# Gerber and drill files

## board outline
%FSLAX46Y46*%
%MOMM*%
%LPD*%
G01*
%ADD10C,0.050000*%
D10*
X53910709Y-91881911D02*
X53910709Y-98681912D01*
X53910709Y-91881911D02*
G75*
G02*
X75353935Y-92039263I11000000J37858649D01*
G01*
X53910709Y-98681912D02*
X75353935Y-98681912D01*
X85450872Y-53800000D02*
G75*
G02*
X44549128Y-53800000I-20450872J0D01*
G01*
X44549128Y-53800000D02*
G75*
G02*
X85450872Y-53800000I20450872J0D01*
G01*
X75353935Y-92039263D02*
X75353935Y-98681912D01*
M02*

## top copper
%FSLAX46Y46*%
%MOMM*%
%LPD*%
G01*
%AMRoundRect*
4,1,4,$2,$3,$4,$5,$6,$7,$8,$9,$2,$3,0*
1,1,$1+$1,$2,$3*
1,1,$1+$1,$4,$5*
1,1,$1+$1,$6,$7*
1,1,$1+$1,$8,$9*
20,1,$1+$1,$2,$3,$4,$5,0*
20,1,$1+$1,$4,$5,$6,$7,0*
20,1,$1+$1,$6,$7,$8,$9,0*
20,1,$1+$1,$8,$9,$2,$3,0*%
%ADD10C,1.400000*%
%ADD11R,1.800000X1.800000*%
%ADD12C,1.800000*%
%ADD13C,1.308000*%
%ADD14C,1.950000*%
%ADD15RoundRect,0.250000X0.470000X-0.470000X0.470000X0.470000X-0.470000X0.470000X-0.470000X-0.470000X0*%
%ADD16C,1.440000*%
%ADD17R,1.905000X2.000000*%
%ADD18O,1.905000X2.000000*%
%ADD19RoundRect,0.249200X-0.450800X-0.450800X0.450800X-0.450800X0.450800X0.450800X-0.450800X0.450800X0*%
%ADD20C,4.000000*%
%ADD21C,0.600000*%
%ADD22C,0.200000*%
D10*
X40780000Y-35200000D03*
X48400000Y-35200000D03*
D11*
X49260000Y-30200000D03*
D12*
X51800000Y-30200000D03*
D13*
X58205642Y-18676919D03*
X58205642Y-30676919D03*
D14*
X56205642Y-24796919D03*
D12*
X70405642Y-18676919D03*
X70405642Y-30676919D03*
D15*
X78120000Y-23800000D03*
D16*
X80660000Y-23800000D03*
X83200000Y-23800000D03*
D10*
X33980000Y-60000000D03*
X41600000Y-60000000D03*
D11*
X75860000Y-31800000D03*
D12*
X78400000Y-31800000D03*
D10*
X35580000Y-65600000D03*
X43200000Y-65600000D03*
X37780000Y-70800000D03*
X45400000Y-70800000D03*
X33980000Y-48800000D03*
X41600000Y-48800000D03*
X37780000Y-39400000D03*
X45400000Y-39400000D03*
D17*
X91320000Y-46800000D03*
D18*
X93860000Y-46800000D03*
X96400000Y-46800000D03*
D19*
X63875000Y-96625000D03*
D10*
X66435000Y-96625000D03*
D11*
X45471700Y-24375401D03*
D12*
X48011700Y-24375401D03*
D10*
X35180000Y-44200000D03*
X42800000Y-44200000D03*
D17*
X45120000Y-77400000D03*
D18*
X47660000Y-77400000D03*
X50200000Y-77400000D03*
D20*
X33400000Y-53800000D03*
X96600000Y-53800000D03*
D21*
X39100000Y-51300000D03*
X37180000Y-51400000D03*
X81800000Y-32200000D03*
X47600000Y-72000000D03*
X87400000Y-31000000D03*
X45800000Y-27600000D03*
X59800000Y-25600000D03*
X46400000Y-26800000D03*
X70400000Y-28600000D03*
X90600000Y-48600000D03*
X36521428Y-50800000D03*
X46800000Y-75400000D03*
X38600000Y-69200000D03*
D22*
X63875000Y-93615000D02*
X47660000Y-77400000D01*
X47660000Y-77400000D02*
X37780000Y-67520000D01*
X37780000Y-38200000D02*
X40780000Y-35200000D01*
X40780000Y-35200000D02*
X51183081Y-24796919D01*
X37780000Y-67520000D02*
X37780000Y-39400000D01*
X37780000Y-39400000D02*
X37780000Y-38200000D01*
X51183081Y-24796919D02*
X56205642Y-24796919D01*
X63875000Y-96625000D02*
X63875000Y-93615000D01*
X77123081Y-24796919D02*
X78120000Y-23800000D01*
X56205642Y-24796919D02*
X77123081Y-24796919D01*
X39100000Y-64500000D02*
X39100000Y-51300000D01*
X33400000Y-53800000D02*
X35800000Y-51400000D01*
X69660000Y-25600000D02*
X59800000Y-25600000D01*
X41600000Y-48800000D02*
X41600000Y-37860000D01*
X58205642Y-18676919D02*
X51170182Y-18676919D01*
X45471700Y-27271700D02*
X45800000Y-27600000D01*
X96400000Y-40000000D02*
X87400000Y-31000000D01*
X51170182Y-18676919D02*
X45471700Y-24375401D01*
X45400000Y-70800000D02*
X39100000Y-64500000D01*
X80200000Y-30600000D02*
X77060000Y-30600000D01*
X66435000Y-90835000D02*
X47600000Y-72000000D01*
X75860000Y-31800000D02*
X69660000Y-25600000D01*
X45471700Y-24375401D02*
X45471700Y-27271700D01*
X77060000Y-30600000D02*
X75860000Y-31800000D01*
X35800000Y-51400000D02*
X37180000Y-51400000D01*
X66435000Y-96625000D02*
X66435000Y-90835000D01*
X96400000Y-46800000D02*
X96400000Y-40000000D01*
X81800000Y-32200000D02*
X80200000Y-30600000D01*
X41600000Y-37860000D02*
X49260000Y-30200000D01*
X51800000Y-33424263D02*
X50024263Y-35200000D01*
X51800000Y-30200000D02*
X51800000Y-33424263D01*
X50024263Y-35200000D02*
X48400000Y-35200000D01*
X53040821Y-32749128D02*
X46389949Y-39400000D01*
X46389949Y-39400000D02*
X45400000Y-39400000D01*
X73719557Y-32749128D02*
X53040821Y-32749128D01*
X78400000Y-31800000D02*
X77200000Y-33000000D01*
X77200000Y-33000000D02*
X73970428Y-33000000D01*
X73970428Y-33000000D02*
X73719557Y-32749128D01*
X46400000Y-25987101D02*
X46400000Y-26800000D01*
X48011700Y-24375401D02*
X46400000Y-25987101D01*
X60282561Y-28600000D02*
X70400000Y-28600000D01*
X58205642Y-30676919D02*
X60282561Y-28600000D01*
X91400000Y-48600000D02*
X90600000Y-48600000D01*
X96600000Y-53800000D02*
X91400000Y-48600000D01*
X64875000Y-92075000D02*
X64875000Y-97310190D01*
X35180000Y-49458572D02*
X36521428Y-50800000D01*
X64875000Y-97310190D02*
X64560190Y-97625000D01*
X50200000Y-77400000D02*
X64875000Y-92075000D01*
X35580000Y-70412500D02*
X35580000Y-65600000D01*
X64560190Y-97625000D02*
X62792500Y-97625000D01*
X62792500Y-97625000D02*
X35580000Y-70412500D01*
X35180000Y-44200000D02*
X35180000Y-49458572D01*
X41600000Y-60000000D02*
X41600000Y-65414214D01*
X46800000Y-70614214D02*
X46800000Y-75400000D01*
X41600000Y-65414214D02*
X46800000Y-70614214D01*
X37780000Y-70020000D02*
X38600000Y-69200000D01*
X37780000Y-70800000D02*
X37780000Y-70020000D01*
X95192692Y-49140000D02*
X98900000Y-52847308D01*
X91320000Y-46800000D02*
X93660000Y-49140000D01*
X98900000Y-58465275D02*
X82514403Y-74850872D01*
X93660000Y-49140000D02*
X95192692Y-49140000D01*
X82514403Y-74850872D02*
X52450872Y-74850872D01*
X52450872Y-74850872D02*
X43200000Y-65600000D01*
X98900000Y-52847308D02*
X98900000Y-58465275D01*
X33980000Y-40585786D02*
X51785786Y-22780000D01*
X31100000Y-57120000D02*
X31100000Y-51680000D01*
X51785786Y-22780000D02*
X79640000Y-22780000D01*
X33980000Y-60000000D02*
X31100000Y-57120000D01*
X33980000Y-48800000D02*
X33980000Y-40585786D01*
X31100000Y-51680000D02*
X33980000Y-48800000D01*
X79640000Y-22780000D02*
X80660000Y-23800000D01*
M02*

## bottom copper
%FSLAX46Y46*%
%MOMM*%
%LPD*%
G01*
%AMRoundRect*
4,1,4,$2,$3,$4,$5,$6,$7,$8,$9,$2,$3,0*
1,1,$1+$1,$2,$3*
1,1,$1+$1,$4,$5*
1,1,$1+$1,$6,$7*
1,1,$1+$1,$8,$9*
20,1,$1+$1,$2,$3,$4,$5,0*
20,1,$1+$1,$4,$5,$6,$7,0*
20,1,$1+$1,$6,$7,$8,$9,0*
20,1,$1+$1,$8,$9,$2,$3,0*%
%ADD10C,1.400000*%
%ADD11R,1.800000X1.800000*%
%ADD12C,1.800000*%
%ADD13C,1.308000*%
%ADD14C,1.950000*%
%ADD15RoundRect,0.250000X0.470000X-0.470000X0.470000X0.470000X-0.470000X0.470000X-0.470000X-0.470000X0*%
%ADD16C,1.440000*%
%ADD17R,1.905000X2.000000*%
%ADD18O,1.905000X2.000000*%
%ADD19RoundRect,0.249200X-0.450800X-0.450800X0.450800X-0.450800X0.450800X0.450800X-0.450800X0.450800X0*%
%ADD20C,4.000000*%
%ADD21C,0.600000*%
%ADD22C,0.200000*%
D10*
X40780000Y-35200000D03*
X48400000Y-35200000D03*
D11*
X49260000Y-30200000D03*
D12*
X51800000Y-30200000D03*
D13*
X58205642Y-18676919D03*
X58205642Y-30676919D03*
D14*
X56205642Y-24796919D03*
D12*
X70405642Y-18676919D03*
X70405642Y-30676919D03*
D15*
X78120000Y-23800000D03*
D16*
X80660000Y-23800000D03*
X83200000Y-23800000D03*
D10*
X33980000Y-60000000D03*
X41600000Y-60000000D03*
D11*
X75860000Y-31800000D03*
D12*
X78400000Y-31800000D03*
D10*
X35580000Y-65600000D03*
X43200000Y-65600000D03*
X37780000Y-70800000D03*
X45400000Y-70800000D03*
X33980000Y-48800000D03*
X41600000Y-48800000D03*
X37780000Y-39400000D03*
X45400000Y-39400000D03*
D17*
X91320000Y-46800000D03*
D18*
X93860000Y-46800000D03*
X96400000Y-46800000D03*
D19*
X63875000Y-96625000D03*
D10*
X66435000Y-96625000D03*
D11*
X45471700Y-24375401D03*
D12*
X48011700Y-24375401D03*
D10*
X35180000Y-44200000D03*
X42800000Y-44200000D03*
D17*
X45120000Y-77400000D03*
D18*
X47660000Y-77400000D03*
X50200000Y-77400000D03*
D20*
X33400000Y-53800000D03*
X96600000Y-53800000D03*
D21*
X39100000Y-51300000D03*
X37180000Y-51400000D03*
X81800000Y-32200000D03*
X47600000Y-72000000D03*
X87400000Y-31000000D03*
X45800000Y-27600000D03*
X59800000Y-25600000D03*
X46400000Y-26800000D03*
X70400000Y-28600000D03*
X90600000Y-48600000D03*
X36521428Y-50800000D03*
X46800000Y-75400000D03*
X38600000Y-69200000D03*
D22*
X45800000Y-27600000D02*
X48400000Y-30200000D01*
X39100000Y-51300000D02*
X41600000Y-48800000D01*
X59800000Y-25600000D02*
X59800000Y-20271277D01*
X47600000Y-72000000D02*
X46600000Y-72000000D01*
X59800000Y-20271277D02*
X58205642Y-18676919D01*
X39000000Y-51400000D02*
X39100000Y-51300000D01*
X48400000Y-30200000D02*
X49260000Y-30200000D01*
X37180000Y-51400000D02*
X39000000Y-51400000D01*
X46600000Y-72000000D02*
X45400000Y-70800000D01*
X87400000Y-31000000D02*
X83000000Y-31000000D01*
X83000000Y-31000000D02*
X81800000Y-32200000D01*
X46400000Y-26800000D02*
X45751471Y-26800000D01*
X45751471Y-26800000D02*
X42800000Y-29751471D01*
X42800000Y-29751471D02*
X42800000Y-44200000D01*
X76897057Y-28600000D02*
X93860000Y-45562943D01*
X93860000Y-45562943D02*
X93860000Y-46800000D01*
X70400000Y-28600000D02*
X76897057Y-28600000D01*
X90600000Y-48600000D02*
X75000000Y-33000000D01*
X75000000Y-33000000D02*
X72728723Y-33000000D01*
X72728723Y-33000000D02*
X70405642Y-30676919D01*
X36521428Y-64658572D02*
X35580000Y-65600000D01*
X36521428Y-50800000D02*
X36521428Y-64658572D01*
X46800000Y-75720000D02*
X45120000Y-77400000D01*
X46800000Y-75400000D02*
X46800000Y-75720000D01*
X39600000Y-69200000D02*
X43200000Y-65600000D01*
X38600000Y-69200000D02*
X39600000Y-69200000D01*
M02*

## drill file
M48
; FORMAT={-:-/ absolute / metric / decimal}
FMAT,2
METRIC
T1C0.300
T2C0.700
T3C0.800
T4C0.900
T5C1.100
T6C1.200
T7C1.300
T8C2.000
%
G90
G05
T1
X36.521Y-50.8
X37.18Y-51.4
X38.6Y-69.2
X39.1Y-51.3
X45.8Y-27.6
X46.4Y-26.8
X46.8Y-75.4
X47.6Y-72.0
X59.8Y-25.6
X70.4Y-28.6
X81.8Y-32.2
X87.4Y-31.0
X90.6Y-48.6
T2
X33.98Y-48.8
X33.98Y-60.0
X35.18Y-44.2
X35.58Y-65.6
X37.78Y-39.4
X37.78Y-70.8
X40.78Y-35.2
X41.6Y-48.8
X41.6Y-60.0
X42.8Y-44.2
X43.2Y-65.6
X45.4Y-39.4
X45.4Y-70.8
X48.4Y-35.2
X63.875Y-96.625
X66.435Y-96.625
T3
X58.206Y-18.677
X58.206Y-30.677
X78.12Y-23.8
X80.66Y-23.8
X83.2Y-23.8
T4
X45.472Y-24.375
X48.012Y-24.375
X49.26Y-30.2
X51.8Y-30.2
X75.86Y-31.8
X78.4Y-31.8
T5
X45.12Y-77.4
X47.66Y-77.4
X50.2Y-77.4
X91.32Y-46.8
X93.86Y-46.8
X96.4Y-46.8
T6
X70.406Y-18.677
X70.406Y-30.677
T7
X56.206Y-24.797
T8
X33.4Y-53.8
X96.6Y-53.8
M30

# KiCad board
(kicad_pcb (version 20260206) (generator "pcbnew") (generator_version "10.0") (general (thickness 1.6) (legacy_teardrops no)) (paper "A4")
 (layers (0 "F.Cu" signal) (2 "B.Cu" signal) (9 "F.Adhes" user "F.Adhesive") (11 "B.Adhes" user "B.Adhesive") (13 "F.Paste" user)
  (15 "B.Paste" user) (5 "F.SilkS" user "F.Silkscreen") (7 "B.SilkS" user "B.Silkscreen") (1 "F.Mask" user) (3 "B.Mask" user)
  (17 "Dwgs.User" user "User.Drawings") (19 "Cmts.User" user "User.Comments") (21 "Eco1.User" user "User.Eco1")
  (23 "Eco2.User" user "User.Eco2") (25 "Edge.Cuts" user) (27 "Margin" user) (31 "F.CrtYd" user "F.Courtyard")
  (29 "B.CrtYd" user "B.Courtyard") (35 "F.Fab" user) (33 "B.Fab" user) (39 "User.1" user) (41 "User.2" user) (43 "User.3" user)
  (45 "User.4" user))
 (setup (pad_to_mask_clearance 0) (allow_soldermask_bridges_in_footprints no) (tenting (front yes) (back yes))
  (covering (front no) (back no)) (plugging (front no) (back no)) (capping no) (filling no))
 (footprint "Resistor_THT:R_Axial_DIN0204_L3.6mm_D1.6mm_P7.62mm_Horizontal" (layer "F.Cu") (at 40.78 35.2)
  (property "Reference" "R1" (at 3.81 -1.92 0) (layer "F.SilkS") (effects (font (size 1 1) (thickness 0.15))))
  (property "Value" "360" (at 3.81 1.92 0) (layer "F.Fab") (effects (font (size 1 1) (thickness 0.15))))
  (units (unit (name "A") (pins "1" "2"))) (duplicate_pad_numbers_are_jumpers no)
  (pad "1" thru_hole circle (at 0 0) (size 1.4 1.4) (drill 0.7) (layers "*.Cu" "*.Mask") (remove_unused_layers no) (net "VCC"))
  (pad "2" thru_hole circle (at 7.62 0) (size 1.4 1.4) (drill 0.7) (layers "*.Cu" "*.Mask") (remove_unused_layers no) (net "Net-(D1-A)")))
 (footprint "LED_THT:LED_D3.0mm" (layer "F.Cu") (at 49.26 30.2)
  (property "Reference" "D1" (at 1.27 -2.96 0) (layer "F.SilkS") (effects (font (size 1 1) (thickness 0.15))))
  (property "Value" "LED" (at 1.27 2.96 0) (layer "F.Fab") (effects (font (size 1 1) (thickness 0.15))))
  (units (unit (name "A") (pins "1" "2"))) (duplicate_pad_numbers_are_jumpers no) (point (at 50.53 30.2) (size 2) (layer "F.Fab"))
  (pad "1" thru_hole rect (at 0 0) (size 1.8 1.8) (drill 0.9) (layers "*.Cu" "*.Mask") (remove_unused_layers no) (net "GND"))
  (pad "2" thru_hole circle (at 2.54 0) (size 1.8 1.8) (drill 0.9) (layers "*.Cu" "*.Mask") (remove_unused_layers no) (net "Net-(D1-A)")))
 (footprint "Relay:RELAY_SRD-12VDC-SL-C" (layer "F.Cu") (at 64.305642 24.676919)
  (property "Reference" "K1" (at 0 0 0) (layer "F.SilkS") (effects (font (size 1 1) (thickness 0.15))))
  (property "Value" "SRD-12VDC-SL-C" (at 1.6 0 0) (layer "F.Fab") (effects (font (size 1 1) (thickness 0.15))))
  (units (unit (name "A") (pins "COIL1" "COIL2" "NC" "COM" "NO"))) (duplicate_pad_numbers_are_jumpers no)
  (pad "COIL1" thru_hole circle (at -6.1 -6) (size 1.308 1.308) (drill 0.8) (layers "*.Cu" "*.Mask") (remove_unused_layers no) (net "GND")
   (solder_mask_margin 0.102))
  (pad "COIL2" thru_hole circle (at -6.1 6) (size 1.308 1.308) (drill 0.8) (layers "*.Cu" "*.Mask") (remove_unused_layers no)
   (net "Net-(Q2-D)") (solder_mask_margin 0.102))
  (pad "COM" thru_hole circle (at -8.1 0.12) (size 1.95 1.95) (drill 1.3) (layers "*.Cu" "*.Mask") (remove_unused_layers no) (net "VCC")
   (solder_mask_margin 0.102))
  (pad "NC" thru_hole circle (at 6.1 -6) (size 1.8 1.8) (drill 1.2) (layers "*.Cu" "*.Mask") (remove_unused_layers no)
   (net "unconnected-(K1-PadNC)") (solder_mask_margin 0.102))
  (pad "NO" thru_hole circle (at 6.1 6) (size 1.8 1.8) (drill 1.2) (layers "*.Cu" "*.Mask") (remove_unused_layers no) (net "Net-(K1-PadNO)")
   (solder_mask_margin 0.102)))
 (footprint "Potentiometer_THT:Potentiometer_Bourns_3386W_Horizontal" (layer "F.Cu") (at 78.12 23.8)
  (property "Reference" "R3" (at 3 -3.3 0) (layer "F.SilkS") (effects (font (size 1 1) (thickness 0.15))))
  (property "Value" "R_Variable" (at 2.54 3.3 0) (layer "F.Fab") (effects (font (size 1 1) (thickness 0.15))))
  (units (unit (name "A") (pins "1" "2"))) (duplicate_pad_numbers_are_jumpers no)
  (pad "1" thru_hole roundrect (at 0 0 90) (size 1.44 1.44) (drill 0.8) (layers "*.Cu" "*.Mask") (remove_unused_layers no)
   (roundrect_rratio 0.1736111111) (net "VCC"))
  (pad "2" thru_hole circle (at 2.54 0 90) (size 1.44 1.44) (drill 0.8) (layers "*.Cu" "*.Mask") (remove_unused_layers no)
   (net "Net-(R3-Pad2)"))
  (pad "3" thru_hole circle (at 5.08 0 90) (size 1.44 1.44) (drill 0.8) (layers "*.Cu" "*.Mask") (remove_unused_layers no)))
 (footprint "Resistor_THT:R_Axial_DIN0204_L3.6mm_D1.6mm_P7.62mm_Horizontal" (layer "F.Cu") (at 33.98 60)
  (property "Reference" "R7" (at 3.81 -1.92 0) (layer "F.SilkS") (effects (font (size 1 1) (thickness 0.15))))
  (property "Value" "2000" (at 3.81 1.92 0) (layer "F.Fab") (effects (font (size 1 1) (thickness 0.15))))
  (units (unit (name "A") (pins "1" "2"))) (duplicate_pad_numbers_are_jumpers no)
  (pad "1" thru_hole circle (at 0 0) (size 1.4 1.4) (drill 0.7) (layers "*.Cu" "*.Mask") (remove_unused_layers no) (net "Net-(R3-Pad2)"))
  (pad "2" thru_hole circle (at 7.62 0) (size 1.4 1.4) (drill 0.7) (layers "*.Cu" "*.Mask") (remove_unused_layers no) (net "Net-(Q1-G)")))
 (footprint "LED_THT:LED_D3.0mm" (layer "F.Cu") (at 75.86 31.8)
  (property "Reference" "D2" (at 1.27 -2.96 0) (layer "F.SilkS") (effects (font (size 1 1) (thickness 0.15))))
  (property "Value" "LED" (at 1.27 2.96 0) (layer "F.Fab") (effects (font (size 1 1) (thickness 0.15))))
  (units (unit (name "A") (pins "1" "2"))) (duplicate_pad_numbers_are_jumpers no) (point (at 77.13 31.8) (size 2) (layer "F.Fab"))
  (pad "1" thru_hole rect (at 0 0) (size 1.8 1.8) (drill 0.9) (layers "*.Cu" "*.Mask") (remove_unused_layers no) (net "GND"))
  (pad "2" thru_hole circle (at 2.54 0) (size 1.8 1.8) (drill 0.9) (layers "*.Cu" "*.Mask") (remove_unused_layers no) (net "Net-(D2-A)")))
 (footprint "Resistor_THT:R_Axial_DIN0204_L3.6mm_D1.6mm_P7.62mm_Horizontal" (layer "F.Cu") (at 35.58 65.6)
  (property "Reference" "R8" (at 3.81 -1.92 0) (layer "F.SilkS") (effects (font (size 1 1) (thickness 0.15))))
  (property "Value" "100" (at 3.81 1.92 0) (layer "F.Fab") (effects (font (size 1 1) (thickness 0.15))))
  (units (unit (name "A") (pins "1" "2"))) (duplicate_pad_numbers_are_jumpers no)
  (pad "1" thru_hole circle (at 0 0) (size 1.4 1.4) (drill 0.7) (layers "*.Cu" "*.Mask") (remove_unused_layers no) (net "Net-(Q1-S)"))
  (pad "2" thru_hole circle (at 7.62 0) (size 1.4 1.4) (drill 0.7) (layers "*.Cu" "*.Mask") (remove_unused_layers no) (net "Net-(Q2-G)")))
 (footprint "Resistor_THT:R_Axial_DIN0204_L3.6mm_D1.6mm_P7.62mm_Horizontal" (layer "F.Cu") (at 37.78 70.8)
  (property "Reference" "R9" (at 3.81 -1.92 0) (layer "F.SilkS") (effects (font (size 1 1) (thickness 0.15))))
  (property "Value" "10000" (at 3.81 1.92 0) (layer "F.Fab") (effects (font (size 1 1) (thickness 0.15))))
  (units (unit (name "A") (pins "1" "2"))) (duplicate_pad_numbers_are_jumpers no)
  (pad "1" thru_hole circle (at 0 0) (size 1.4 1.4) (drill 0.7) (layers "*.Cu" "*.Mask") (remove_unused_layers no) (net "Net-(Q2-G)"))
  (pad "2" thru_hole circle (at 7.62 0) (size 1.4 1.4) (drill 0.7) (layers "*.Cu" "*.Mask") (remove_unused_layers no) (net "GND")))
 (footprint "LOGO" (layer "F.Cu") (at 91 68.8 90)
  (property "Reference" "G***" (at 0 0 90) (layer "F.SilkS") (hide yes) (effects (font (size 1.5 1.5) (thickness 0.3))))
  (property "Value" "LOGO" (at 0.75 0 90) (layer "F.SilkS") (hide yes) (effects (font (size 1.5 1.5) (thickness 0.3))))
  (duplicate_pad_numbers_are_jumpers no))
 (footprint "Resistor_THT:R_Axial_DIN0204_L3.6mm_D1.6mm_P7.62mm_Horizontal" (layer "F.Cu") (at 33.98 48.8)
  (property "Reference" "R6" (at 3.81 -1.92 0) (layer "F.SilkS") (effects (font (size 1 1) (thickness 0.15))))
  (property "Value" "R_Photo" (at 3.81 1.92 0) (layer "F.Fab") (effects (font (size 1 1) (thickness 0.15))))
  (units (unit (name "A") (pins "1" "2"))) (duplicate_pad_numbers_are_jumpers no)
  (pad "1" thru_hole circle (at 0 0) (size 1.4 1.4) (drill 0.7) (layers "*.Cu" "*.Mask") (remove_unused_layers no) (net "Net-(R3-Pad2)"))
  (pad "2" thru_hole circle (at 7.62 0) (size 1.4 1.4) (drill 0.7) (layers "*.Cu" "*.Mask") (remove_unused_layers no) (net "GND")))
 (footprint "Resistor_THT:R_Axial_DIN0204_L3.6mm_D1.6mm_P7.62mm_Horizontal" (layer "F.Cu") (at 37.78 39.4)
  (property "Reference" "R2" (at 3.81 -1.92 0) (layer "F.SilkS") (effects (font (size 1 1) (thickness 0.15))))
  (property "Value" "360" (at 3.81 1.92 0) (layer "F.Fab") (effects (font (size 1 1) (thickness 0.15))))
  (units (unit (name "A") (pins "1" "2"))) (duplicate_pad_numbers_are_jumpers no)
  (pad "1" thru_hole circle (at 0 0) (size 1.4 1.4) (drill 0.7) (layers "*.Cu" "*.Mask") (remove_unused_layers no) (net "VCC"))
  (pad "2" thru_hole circle (at 7.62 0) (size 1.4 1.4) (drill 0.7) (layers "*.Cu" "*.Mask") (remove_unused_layers no) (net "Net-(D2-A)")))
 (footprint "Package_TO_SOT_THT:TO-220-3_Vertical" (layer "F.Cu") (at 91.32 46.8)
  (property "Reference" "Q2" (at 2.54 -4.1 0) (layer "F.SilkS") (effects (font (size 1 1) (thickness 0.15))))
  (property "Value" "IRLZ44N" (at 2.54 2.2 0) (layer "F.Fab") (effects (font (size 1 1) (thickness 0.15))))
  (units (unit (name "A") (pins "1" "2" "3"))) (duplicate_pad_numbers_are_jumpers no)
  (pad "1" thru_hole rect (at 0 0) (size 1.905 2) (drill 1.1) (layers "*.Cu" "*.Mask") (remove_unused_layers no) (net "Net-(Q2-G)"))
  (pad "2" thru_hole oval (at 2.54 0) (size 1.905 2) (drill 1.1) (layers "*.Cu" "*.Mask") (remove_unused_layers no) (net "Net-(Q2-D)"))
  (pad "3" thru_hole oval (at 5.08 0) (size 1.905 2) (drill 1.1) (layers "*.Cu" "*.Mask") (remove_unused_layers no) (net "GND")))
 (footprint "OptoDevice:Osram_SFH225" (layer "F.Cu") (at 63.875 96.625)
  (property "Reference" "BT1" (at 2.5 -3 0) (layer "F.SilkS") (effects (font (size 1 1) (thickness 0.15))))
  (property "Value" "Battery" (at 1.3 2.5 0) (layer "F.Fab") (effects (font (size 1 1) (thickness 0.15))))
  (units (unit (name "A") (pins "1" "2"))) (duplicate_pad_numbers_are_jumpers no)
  (pad "1" thru_hole roundrect (at 0 0) (size 1.4 1.4) (drill 0.7) (layers "*.Cu" "*.Mask") (remove_unused_layers no)
   (roundrect_rratio 0.178) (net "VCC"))
  (pad "2" thru_hole circle (at 2.56 0) (size 1.4 1.4) (drill 0.7) (layers "*.Cu" "*.Mask") (remove_unused_layers no) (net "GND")))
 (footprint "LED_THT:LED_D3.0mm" (layer "F.Cu") (at 45.4717 24.375401)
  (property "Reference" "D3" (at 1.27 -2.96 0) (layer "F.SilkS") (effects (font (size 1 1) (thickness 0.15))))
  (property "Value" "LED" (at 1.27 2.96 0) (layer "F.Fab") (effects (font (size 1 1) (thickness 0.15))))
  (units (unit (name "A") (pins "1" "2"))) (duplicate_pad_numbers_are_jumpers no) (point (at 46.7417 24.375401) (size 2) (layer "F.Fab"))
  (pad "1" thru_hole rect (at 0 0) (size 1.8 1.8) (drill 0.9) (layers "*.Cu" "*.Mask") (remove_unused_layers no) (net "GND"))
  (pad "2" thru_hole circle (at 2.54 0) (size 1.8 1.8) (drill 0.9) (layers "*.Cu" "*.Mask") (remove_unused_layers no) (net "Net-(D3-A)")))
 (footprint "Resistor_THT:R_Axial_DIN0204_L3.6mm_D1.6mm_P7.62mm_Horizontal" (layer "F.Cu") (at 35.18 44.2)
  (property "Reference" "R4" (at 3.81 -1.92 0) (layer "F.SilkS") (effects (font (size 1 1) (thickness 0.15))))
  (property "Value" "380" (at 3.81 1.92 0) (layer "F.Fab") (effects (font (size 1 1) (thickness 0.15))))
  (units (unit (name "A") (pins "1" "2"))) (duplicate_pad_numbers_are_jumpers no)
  (pad "1" thru_hole circle (at 0 0) (size 1.4 1.4) (drill 0.7) (layers "*.Cu" "*.Mask") (remove_unused_layers no) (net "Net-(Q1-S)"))
  (pad "2" thru_hole circle (at 7.62 0) (size 1.4 1.4) (drill 0.7) (layers "*.Cu" "*.Mask") (remove_unused_layers no) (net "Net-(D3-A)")))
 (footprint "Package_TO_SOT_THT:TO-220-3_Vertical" (layer "F.Cu") (at 45.12 77.4)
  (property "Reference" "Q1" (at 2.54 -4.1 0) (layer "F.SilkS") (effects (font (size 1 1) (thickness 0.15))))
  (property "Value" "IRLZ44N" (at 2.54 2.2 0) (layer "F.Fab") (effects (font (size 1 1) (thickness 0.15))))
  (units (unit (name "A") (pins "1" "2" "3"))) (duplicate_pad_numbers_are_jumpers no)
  (pad "1" thru_hole rect (at 0 0) (size 1.905 2) (drill 1.1) (layers "*.Cu" "*.Mask") (remove_unused_layers no) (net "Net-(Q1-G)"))
  (pad "2" thru_hole oval (at 2.54 0) (size 1.905 2) (drill 1.1) (layers "*.Cu" "*.Mask") (remove_unused_layers no) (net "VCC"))
  (pad "3" thru_hole oval (at 5.08 0) (size 1.905 2) (drill 1.1) (layers "*.Cu" "*.Mask") (remove_unused_layers no) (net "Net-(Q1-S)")))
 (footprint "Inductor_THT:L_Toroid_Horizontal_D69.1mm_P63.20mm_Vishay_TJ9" (layer "F.Cu") (at 33.4 53.8)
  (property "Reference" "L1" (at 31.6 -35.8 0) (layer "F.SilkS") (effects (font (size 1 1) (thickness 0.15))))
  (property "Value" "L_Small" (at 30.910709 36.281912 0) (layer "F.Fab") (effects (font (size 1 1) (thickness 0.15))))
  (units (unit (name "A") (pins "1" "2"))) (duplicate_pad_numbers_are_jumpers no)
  (pad "1" thru_hole circle (at 0 0) (size 4 4) (drill 2) (layers "*.Cu" "*.Mask") (remove_unused_layers no) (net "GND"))
  (pad "2" thru_hole circle (at 63.2 0) (size 4 4) (drill 2) (layers "*.Cu" "*.Mask") (remove_unused_layers no) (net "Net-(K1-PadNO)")))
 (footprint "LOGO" (layer "F.Cu") (at 65 86.945401)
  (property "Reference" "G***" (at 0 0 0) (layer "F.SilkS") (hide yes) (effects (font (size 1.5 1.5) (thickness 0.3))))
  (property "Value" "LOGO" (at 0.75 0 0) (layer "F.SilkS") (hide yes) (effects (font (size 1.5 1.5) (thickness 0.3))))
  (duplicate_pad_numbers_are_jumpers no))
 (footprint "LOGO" (layer "F.Cu") (at 88.44957 36.320805)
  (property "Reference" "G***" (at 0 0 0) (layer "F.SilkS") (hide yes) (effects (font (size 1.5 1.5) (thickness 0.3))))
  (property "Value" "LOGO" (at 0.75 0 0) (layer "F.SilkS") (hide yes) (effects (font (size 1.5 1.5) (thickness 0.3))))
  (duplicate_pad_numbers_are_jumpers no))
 (gr_line (start 53.910709 91.881911) (end 53.910709 98.681912) (stroke (width 0.05) (type default)) (layer "Edge.Cuts"))
 (gr_arc (start 53.910709 91.881911) (mid 65.2 14.6) (end 75.353935 92.039263) (stroke (width 0.05) (type default)) (layer "Edge.Cuts"))
 (gr_line (start 53.910709 98.681912) (end 75.353935 98.681912) (stroke (width 0.05) (type default)) (layer "Edge.Cuts"))
 (gr_circle (center 65 53.8) (end 71.004308 73.34959) (stroke (width 0.05) (type default)) (fill no) (layer "Edge.Cuts"))
 (gr_line (start 75.353935 92.039263) (end 75.353935 98.681912) (stroke (width 0.05) (type default)) (layer "Edge.Cuts"))
 (segment (start 63.875 93.615) (end 47.66 77.4) (width 0.2) (layer "F.Cu") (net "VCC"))
 (segment (start 47.66 77.4) (end 37.78 67.52) (width 0.2) (layer "F.Cu") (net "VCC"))
 (segment (start 37.78 38.2) (end 40.78 35.2) (width 0.2) (layer "F.Cu") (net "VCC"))
 (segment (start 40.78 35.2) (end 51.183081 24.796919) (width 0.2) (layer "F.Cu") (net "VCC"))
 (segment (start 37.78 67.52) (end 37.78 39.4) (width 0.2) (layer "F.Cu") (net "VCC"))
 (segment (start 37.78 39.4) (end 37.78 38.2) (width 0.2) (layer "F.Cu") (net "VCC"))
 (segment (start 51.183081 24.796919) (end 56.205642 24.796919) (width 0.2) (layer "F.Cu") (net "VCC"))
 (segment (start 63.875 96.625) (end 63.875 93.615) (width 0.2) (layer "F.Cu") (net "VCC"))
 (segment (start 77.123081 24.796919) (end 78.12 23.8) (width 0.2) (layer "F.Cu") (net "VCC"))
 (segment (start 56.205642 24.796919) (end 77.123081 24.796919) (width 0.2) (layer "F.Cu") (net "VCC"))
 (segment (start 39.1 64.5) (end 39.1 51.3) (width 0.2) (layer "F.Cu") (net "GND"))
 (segment (start 33.4 53.8) (end 35.8 51.4) (width 0.2) (layer "F.Cu") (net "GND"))
 (segment (start 69.66 25.6) (end 59.8 25.6) (width 0.2) (layer "F.Cu") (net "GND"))
 (segment (start 41.6 48.8) (end 41.6 37.86) (width 0.2) (layer "F.Cu") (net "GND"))
 (segment (start 58.205642 18.676919) (end 51.170182 18.676919) (width 0.2) (layer "F.Cu") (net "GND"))
 (segment (start 45.4717 27.2717) (end 45.8 27.6) (width 0.2) (layer "F.Cu") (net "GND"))
 (segment (start 96.4 40) (end 87.4 31) (width 0.2) (layer "F.Cu") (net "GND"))
 (segment (start 51.170182 18.676919) (end 45.4717 24.375401) (width 0.2) (layer "F.Cu") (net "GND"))
 (segment (start 45.4 70.8) (end 39.1 64.5) (width 0.2) (layer "F.Cu") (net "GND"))
 (segment (start 80.2 30.6) (end 77.06 30.6) (width 0.2) (layer "F.Cu") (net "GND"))
 (segment (start 66.435 90.835) (end 47.6 72) (width 0.2) (layer "F.Cu") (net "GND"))
 (segment (start 75.86 31.8) (end 69.66 25.6) (width 0.2) (layer "F.Cu") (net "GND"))
 (segment (start 45.4717 24.375401) (end 45.4717 27.2717) (width 0.2) (layer "F.Cu") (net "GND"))
 (segment (start 77.06 30.6) (end 75.86 31.8) (width 0.2) (layer "F.Cu") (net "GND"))
 (segment (start 35.8 51.4) (end 37.18 51.4) (width 0.2) (layer "F.Cu") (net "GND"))
 (segment (start 66.435 96.625) (end 66.435 90.835) (width 0.2) (layer "F.Cu") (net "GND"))
 (segment (start 96.4 46.8) (end 96.4 40) (width 0.2) (layer "F.Cu") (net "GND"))
 (segment (start 81.8 32.2) (end 80.2 30.6) (width 0.2) (layer "F.Cu") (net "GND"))
 (segment (start 41.6 37.86) (end 49.26 30.2) (width 0.2) (layer "F.Cu") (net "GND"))
 (via (at 39.1 51.3) (size 0.6) (drill 0.3) (layers "F.Cu" "B.Cu") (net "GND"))
 (via (at 37.18 51.4) (size 0.6) (drill 0.3) (layers "F.Cu" "B.Cu") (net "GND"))
 (via (at 81.8 32.2) (size 0.6) (drill 0.3) (layers "F.Cu" "B.Cu") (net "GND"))
 (via (at 47.6 72) (size 0.6) (drill 0.3) (layers "F.Cu" "B.Cu") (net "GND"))
 (via (at 87.4 31) (size 0.6) (drill 0.3) (layers "F.Cu" "B.Cu") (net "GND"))
 (via (at 45.8 27.6) (size 0.6) (drill 0.3) (layers "F.Cu" "B.Cu") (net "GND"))
 (via (at 59.8 25.6) (size 0.6) (drill 0.3) (layers "F.Cu" "B.Cu") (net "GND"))
 (segment (start 45.8 27.6) (end 48.4 30.2) (width 0.2) (layer "B.Cu") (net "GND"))
 (segment (start 39.1 51.3) (end 41.6 48.8) (width 0.2) (layer "B.Cu") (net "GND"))
 (segment (start 59.8 25.6) (end 59.8 20.271277) (width 0.2) (layer "B.Cu") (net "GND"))
 (segment (start 47.6 72) (end 46.6 72) (width 0.2) (layer "B.Cu") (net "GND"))
 (segment (start 59.8 20.271277) (end 58.205642 18.676919) (width 0.2) (layer "B.Cu") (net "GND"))
 (segment (start 39 51.4) (end 39.1 51.3) (width 0.2) (layer "B.Cu") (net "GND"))
 (segment (start 48.4 30.2) (end 49.26 30.2) (width 0.2) (layer "B.Cu") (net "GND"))
 (segment (start 37.18 51.4) (end 39 51.4) (width 0.2) (layer "B.Cu") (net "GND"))
 (segment (start 46.6 72) (end 45.4 70.8) (width 0.2) (layer "B.Cu") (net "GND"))
 (segment (start 87.4 31) (end 83 31) (width 0.2) (layer "B.Cu") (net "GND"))
 (segment (start 83 31) (end 81.8 32.2) (width 0.2) (layer "B.Cu") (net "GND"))
 (segment (start 51.8 33.424263) (end 50.024263 35.2) (width 0.2) (layer "F.Cu") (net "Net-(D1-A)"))
 (segment (start 51.8 30.2) (end 51.8 33.424263) (width 0.2) (layer "F.Cu") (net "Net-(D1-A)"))
 (segment (start 50.024263 35.2) (end 48.4 35.2) (width 0.2) (layer "F.Cu") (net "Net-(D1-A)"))
 (segment (start 53.040821 32.749128) (end 46.389949 39.4) (width 0.2) (layer "F.Cu") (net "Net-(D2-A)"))
 (segment (start 46.389949 39.4) (end 45.4 39.4) (width 0.2) (layer "F.Cu") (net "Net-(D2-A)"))
 (segment (start 73.719557 32.749128) (end 53.040821 32.749128) (width 0.2) (layer "F.Cu") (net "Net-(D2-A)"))
 (segment (start 78.4 31.8) (end 77.2 33) (width 0.2) (layer "F.Cu") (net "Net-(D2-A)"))
 (segment (start 77.2 33) (end 73.970428 33) (width 0.2) (layer "F.Cu") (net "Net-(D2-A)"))
 (segment (start 73.970428 33) (end 73.719557 32.749128) (width 0.2) (layer "F.Cu") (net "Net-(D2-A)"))
 (segment (start 46.4 25.987101) (end 46.4 26.8) (width 0.2) (layer "F.Cu") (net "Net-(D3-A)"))
 (segment (start 48.0117 24.375401) (end 46.4 25.987101) (width 0.2) (layer "F.Cu") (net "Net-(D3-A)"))
 (via (at 46.4 26.8) (size 0.6) (drill 0.3) (layers "F.Cu" "B.Cu") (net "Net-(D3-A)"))
 (segment (start 46.4 26.8) (end 45.751471 26.8) (width 0.2) (layer "B.Cu") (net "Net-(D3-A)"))
 (segment (start 45.751471 26.8) (end 42.8 29.751471) (width 0.2) (layer "B.Cu") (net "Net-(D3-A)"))
 (segment (start 42.8 29.751471) (end 42.8 44.2) (width 0.2) (layer "B.Cu") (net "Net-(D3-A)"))
 (segment (start 60.282561 28.6) (end 70.4 28.6) (width 0.2) (layer "F.Cu") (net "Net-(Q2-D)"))
 (segment (start 58.205642 30.676919) (end 60.282561 28.6) (width 0.2) (layer "F.Cu") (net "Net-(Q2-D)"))
 (via (at 70.4 28.6) (size 0.6) (drill 0.3) (layers "F.Cu" "B.Cu") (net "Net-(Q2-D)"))
 (segment (start 76.897057 28.6) (end 93.86 45.562943) (width 0.2) (layer "B.Cu") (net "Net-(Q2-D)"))
 (segment (start 93.86 45.562943) (end 93.86 46.8) (width 0.2) (layer "B.Cu") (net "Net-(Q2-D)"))
 (segment (start 70.4 28.6) (end 76.897057 28.6) (width 0.2) (layer "B.Cu") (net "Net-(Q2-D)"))
 (segment (start 91.4 48.6) (end 90.6 48.6) (width 0.2) (layer "F.Cu") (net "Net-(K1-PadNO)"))
 (segment (start 96.6 53.8) (end 91.4 48.6) (width 0.2) (layer "F.Cu") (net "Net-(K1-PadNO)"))
 (via (at 90.6 48.6) (size 0.6) (drill 0.3) (layers "F.Cu" "B.Cu") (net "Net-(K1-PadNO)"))
 (segment (start 90.6 48.6) (end 75 33) (width 0.2) (layer "B.Cu") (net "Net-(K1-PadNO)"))
 (segment (start 75 33) (end 72.728723 33) (width 0.2) (layer "B.Cu") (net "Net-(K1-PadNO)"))
 (segment (start 72.728723 33) (end 70.405642 30.676919) (width 0.2) (layer "B.Cu") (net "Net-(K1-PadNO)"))
 (segment (start 64.875 92.075) (end 64.875 97.31019) (width 0.2) (layer "F.Cu") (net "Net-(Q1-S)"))
 (segment (start 35.18 49.458572) (end 36.521428 50.8) (width 0.2) (layer "F.Cu") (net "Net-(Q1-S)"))
 (segment (start 64.875 97.31019) (end 64.56019 97.625) (width 0.2) (layer "F.Cu") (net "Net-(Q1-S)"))
 (segment (start 50.2 77.4) (end 64.875 92.075) (width 0.2) (layer "F.Cu") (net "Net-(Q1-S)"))
 (segment (start 35.58 70.4125) (end 35.58 65.6) (width 0.2) (layer "F.Cu") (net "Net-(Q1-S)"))
 (segment (start 64.56019 97.625) (end 62.7925 97.625) (width 0.2) (layer "F.Cu") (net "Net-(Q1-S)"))
 (segment (start 62.7925 97.625) (end 35.58 70.4125) (width 0.2) (layer "F.Cu") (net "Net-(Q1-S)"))
 (segment (start 35.18 44.2) (end 35.18 49.458572) (width 0.2) (layer "F.Cu") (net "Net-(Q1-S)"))
 (via (at 36.521428 50.8) (size 0.6) (drill 0.3) (layers "F.Cu" "B.Cu") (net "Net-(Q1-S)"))
 (segment (start 36.521428 64.658572) (end 35.58 65.6) (width 0.2) (layer "B.Cu") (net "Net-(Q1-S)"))
 (segment (start 36.521428 50.8) (end 36.521428 64.658572) (width 0.2) (layer "B.Cu") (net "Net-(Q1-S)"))
 (segment (start 41.6 60) (end 41.6 65.414214) (width 0.2) (layer "F.Cu") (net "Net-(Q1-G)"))
 (segment (start 46.8 70.614214) (end 46.8 75.4) (width 0.2) (layer "F.Cu") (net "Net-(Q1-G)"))
 (segment (start 41.6 65.414214) (end 46.8 70.614214) (width 0.2) (layer "F.Cu") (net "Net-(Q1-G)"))
 (via (at 46.8 75.4) (size 0.6) (drill 0.3) (layers "F.Cu" "B.Cu") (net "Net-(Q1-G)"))
 (segment (start 46.8 75.72) (end 45.12 77.4) (width 0.2) (layer "B.Cu") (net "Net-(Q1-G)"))
 (segment (start 46.8 75.4) (end 46.8 75.72) (width 0.2) (layer "B.Cu") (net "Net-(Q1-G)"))
 (segment (start 37.78 70.02) (end 38.6 69.2) (width 0.2) (layer "F.Cu") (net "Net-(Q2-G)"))
 (segment (start 37.78 70.8) (end 37.78 70.02) (width 0.2) (layer "F.Cu") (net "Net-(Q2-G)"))
 (segment (start 95.192692 49.14) (end 98.9 52.847308) (width 0.2) (layer "F.Cu") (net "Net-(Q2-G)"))
 (segment (start 91.32 46.8) (end 93.66 49.14) (width 0.2) (layer "F.Cu") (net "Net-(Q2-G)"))
 (segment (start 98.9 58.465275) (end 82.514403 74.850872) (width 0.2) (layer "F.Cu") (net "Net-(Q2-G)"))
 (segment (start 93.66 49.14) (end 95.192692 49.14) (width 0.2) (layer "F.Cu") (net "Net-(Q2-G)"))
 (segment (start 82.514403 74.850872) (end 52.450872 74.850872) (width 0.2) (layer "F.Cu") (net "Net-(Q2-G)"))
 (segment (start 52.450872 74.850872) (end 43.2 65.6) (width 0.2) (layer "F.Cu") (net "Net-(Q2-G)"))
 (segment (start 98.9 52.847308) (end 98.9 58.465275) (width 0.2) (layer "F.Cu") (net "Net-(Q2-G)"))
 (via (at 38.6 69.2) (size 0.6) (drill 0.3) (layers "F.Cu" "B.Cu") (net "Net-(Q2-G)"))
 (segment (start 39.6 69.2) (end 43.2 65.6) (width 0.2) (layer "B.Cu") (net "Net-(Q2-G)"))
 (segment (start 38.6 69.2) (end 39.6 69.2) (width 0.2) (layer "B.Cu") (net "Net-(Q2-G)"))
 (segment (start 33.98 40.585786) (end 51.785786 22.78) (width 0.2) (layer "F.Cu") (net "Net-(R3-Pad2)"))
 (segment (start 31.1 57.12) (end 31.1 51.68) (width 0.2) (layer "F.Cu") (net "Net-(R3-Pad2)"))
 (segment (start 51.785786 22.78) (end 79.64 22.78) (width 0.2) (layer "F.Cu") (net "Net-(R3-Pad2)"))
 (segment (start 33.98 60) (end 31.1 57.12) (width 0.2) (layer "F.Cu") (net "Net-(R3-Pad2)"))
 (segment (start 33.98 48.8) (end 33.98 40.585786) (width 0.2) (layer "F.Cu") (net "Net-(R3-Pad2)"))
 (segment (start 31.1 51.68) (end 33.98 48.8) (width 0.2) (layer "F.Cu") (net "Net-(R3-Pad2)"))
 (segment (start 79.64 22.78) (end 80.66 23.8) (width 0.2) (layer "F.Cu") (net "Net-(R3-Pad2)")))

